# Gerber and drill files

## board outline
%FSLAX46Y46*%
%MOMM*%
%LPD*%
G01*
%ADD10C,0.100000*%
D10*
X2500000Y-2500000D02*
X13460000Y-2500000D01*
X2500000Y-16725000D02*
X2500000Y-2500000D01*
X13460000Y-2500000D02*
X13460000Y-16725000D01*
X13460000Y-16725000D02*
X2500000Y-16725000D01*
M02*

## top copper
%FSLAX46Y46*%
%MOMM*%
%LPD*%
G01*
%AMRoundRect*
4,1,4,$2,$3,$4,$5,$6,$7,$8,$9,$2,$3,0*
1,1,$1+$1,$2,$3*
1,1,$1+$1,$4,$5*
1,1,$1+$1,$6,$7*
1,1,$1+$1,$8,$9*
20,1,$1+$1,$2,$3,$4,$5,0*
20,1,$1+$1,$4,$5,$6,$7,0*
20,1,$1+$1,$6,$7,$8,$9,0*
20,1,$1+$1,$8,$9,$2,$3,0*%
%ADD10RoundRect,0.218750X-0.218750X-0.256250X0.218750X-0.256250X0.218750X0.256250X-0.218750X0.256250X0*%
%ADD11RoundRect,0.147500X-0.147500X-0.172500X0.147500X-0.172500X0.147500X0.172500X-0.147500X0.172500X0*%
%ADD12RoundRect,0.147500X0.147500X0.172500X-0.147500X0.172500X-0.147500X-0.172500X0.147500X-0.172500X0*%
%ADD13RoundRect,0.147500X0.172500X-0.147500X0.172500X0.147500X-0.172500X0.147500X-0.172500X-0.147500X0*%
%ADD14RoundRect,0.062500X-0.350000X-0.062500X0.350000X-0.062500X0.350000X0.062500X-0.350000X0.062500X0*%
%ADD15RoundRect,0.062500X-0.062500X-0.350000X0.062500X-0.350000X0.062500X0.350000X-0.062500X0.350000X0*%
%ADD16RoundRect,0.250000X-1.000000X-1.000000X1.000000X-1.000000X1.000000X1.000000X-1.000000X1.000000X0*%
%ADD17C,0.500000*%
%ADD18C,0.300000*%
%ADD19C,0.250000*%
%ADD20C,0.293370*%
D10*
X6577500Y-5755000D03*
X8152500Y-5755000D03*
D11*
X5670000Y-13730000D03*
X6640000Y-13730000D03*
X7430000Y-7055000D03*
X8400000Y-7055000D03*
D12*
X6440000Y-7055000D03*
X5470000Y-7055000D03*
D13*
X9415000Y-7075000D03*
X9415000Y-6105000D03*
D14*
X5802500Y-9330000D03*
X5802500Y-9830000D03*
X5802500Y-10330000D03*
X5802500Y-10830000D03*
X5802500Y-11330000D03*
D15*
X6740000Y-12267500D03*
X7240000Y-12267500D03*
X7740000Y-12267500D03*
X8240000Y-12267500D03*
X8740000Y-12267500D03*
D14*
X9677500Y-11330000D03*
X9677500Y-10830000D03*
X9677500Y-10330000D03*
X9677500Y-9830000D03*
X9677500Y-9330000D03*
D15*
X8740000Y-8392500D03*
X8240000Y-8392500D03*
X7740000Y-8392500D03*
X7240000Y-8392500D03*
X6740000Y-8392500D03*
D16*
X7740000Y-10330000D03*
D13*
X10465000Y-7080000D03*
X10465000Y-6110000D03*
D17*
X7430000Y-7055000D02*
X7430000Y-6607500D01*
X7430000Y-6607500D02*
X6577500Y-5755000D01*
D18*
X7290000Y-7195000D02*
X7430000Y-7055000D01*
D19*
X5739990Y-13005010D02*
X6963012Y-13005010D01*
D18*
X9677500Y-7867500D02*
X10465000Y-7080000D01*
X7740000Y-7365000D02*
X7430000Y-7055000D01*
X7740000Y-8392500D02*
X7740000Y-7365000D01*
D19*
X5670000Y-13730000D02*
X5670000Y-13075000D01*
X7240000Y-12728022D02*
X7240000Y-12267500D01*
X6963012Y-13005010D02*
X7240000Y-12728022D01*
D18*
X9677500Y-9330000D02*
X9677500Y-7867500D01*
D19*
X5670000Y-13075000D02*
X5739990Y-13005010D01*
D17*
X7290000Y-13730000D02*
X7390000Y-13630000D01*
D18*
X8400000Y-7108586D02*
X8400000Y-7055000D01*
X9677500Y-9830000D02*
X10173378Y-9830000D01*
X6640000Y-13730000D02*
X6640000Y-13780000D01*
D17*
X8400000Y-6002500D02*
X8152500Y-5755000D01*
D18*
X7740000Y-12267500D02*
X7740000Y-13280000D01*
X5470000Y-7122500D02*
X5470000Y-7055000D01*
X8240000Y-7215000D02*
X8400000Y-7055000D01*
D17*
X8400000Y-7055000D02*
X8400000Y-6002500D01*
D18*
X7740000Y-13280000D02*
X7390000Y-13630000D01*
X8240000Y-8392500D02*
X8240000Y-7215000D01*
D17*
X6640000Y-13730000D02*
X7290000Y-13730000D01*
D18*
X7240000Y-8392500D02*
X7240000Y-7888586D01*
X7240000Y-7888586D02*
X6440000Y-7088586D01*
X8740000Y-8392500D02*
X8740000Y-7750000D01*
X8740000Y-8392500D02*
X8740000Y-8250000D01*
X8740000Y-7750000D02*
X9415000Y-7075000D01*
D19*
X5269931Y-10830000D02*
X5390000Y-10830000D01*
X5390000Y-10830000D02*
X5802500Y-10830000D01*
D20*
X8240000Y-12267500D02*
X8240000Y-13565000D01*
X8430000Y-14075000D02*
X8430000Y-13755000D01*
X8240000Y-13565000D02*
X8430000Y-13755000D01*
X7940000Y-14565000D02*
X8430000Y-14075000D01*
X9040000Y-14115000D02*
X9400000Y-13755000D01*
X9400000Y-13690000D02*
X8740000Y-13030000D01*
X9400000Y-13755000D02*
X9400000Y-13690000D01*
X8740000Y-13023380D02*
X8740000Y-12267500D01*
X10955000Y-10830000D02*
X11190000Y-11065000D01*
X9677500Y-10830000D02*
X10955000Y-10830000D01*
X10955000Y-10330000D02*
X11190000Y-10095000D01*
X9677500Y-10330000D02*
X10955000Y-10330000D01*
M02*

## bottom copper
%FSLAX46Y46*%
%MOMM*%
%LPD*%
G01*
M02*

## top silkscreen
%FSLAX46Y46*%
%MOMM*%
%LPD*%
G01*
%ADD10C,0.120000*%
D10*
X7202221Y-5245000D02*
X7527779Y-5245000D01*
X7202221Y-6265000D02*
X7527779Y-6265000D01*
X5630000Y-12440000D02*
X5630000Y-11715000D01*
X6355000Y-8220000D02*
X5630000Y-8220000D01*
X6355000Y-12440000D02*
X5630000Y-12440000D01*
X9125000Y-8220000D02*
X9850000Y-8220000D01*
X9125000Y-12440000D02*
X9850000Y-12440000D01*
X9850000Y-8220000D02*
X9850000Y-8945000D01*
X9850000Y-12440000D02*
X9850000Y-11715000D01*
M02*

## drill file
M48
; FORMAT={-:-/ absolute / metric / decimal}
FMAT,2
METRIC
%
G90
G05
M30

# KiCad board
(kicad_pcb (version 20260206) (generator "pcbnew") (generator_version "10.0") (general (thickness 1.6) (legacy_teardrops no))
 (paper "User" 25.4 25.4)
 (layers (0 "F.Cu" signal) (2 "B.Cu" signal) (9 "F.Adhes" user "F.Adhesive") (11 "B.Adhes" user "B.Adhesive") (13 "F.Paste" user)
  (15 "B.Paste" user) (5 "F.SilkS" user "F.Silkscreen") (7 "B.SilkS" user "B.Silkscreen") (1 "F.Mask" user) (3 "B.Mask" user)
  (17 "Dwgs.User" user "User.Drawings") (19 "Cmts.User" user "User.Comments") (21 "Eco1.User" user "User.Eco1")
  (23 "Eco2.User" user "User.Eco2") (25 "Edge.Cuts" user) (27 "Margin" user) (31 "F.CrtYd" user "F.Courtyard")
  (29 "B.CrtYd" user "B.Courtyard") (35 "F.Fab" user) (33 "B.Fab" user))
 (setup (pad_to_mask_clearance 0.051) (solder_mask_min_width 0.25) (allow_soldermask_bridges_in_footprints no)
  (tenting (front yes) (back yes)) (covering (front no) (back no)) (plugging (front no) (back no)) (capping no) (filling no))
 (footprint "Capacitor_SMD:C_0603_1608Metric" (layer "F.Cu") (at 7.365 5.755)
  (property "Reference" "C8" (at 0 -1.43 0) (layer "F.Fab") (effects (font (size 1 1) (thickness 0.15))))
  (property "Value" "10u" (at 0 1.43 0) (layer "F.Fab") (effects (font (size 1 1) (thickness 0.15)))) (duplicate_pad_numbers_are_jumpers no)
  (fp_line (start -0.162779 -0.51) (end 0.162779 -0.51) (stroke (width 0.12) (type solid)) (layer "F.SilkS"))
  (fp_line (start -0.162779 0.51) (end 0.162779 0.51) (stroke (width 0.12) (type solid)) (layer "F.SilkS"))
  (pad "1" smd roundrect (at -0.7875 0) (size 0.875 0.95) (layers "F.Cu" "F.Mask" "F.Paste") (roundrect_rratio 0.25) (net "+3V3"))
  (pad "2" smd roundrect (at 0.7875 0) (size 0.875 0.95) (layers "F.Cu" "F.Mask" "F.Paste") (roundrect_rratio 0.25) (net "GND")))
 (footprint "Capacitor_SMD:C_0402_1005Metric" (layer "F.Cu") (at 6.155 13.73)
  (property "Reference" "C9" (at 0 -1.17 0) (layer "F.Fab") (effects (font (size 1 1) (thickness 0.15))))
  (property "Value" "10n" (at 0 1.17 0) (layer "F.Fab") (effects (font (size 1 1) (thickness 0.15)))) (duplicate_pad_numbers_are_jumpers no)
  (pad "1" smd roundrect (at -0.485 0) (size 0.59 0.64) (layers "F.Cu" "F.Mask" "F.Paste") (roundrect_rratio 0.25) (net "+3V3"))
  (pad "2" smd roundrect (at 0.485 0) (size 0.59 0.64) (layers "F.Cu" "F.Mask" "F.Paste") (roundrect_rratio 0.25) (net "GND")))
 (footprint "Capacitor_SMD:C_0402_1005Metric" (layer "F.Cu") (at 7.915 7.055)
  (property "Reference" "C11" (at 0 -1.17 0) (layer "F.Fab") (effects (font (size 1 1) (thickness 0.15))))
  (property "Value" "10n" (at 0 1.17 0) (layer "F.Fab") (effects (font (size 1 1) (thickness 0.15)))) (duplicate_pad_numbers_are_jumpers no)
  (pad "1" smd roundrect (at -0.485 0) (size 0.59 0.64) (layers "F.Cu" "F.Mask" "F.Paste") (roundrect_rratio 0.25) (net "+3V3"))
  (pad "2" smd roundrect (at 0.485 0) (size 0.59 0.64) (layers "F.Cu" "F.Mask" "F.Paste") (roundrect_rratio 0.25) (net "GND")))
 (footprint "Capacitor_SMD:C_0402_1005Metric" (layer "F.Cu") (at 5.955 7.055 180)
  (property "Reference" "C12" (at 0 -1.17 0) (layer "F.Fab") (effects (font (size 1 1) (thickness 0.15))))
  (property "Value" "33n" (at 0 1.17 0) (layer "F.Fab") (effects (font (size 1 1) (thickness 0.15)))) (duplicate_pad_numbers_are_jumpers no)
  (pad "1" smd roundrect (at -0.485 0 180) (size 0.59 0.64) (layers "F.Cu" "F.Mask" "F.Paste") (roundrect_rratio 0.25)
   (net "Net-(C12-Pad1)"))
  (pad "2" smd roundrect (at 0.485 0 180) (size 0.59 0.64) (layers "F.Cu" "F.Mask" "F.Paste") (roundrect_rratio 0.25) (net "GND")))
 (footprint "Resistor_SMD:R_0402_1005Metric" (layer "F.Cu") (at 9.415 6.59 90)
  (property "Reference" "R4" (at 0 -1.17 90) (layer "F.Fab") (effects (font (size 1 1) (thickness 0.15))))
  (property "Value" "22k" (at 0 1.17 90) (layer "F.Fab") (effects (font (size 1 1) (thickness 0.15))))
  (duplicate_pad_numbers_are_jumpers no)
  (pad "1" smd roundrect (at -0.485 0 90) (size 0.59 0.64) (layers "F.Cu" "F.Mask" "F.Paste") (roundrect_rratio 0.25) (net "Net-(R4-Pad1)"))
  (pad "2" smd roundrect (at 0.485 0 90) (size 0.59 0.64) (layers "F.Cu" "F.Mask" "F.Paste") (roundrect_rratio 0.25) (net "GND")))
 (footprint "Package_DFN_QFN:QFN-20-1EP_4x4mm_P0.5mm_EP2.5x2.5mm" (layer "F.Cu") (at 7.74 10.33)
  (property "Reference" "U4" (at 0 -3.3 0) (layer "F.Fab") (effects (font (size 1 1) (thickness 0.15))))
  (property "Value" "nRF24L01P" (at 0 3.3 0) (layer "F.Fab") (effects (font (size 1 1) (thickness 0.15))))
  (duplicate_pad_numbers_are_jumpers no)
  (fp_line (start -2.11 2.11) (end -2.11 1.385) (stroke (width 0.12) (type solid)) (layer "F.SilkS"))
  (fp_line (start -1.385 -2.11) (end -2.11 -2.11) (stroke (width 0.12) (type solid)) (layer "F.SilkS"))
  (fp_line (start -1.385 2.11) (end -2.11 2.11) (stroke (width 0.12) (type solid)) (layer "F.SilkS"))
  (fp_line (start 1.385 -2.11) (end 2.11 -2.11) (stroke (width 0.12) (type solid)) (layer "F.SilkS"))
  (fp_line (start 1.385 2.11) (end 2.11 2.11) (stroke (width 0.12) (type solid)) (layer "F.SilkS"))
  (fp_line (start 2.11 -2.11) (end 2.11 -1.385) (stroke (width 0.12) (type solid)) (layer "F.SilkS"))
  (fp_line (start 2.11 2.11) (end 2.11 1.385) (stroke (width 0.12) (type solid)) (layer "F.SilkS"))
  (pad "" smd roundrect (at -0.625 -0.625) (size 1.01 1.01) (layers "F.Paste") (roundrect_rratio 0.247525))
  (pad "" smd roundrect (at -0.625 0.625) (size 1.01 1.01) (layers "F.Paste") (roundrect_rratio 0.247525))
  (pad "" smd roundrect (at 0.625 -0.625) (size 1.01 1.01) (layers "F.Paste") (roundrect_rratio 0.247525))
  (pad "" smd roundrect (at 0.625 0.625) (size 1.01 1.01) (layers "F.Paste") (roundrect_rratio 0.247525))
  (pad "1" smd roundrect (at -1.9375 -1) (size 0.825 0.25) (layers "F.Cu" "F.Mask" "F.Paste") (roundrect_rratio 0.25) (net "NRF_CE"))
  (pad "2" smd roundrect (at -1.9375 -0.5) (size 0.825 0.25) (layers "F.Cu" "F.Mask" "F.Paste") (roundrect_rratio 0.25) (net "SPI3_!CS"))
  (pad "3" smd roundrect (at -1.9375 0) (size 0.825 0.25) (layers "F.Cu" "F.Mask" "F.Paste") (roundrect_rratio 0.25) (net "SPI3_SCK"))
  (pad "4" smd roundrect (at -1.9375 0.5) (size 0.825 0.25) (layers "F.Cu" "F.Mask" "F.Paste") (roundrect_rratio 0.25) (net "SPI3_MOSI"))
  (pad "5" smd roundrect (at -1.9375 1) (size 0.825 0.25) (layers "F.Cu" "F.Mask" "F.Paste") (roundrect_rratio 0.25) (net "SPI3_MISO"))
  (pad "6" smd roundrect (at -1 1.9375) (size 0.25 0.825) (layers "F.Cu" "F.Mask" "F.Paste") (roundrect_rratio 0.25) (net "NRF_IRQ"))
  (pad "7" smd roundrect (at -0.5 1.9375) (size 0.25 0.825) (layers "F.Cu" "F.Mask" "F.Paste") (roundrect_rratio 0.25) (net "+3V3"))
  (pad "8" smd roundrect (at 0 1.9375) (size 0.25 0.825) (layers "F.Cu" "F.Mask" "F.Paste") (roundrect_rratio 0.25) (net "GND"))
  (pad "9" smd roundrect (at 0.5 1.9375) (size 0.25 0.825) (layers "F.Cu" "F.Mask" "F.Paste") (roundrect_rratio 0.25) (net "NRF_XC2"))
  (pad "10" smd roundrect (at 1 1.9375) (size 0.25 0.825) (layers "F.Cu" "F.Mask" "F.Paste") (roundrect_rratio 0.25) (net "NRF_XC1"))
  (pad "11" smd roundrect (at 1.9375 1) (size 0.825 0.25) (layers "F.Cu" "F.Mask" "F.Paste") (roundrect_rratio 0.25) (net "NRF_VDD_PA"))
  (pad "12" smd roundrect (at 1.9375 0.5) (size 0.825 0.25) (layers "F.Cu" "F.Mask" "F.Paste") (roundrect_rratio 0.25) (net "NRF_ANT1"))
  (pad "13" smd roundrect (at 1.9375 0) (size 0.825 0.25) (layers "F.Cu" "F.Mask" "F.Paste") (roundrect_rratio 0.25) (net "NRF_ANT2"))
  (pad "14" smd roundrect (at 1.9375 -0.5) (size 0.825 0.25) (layers "F.Cu" "F.Mask" "F.Paste") (roundrect_rratio 0.25) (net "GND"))
  (pad "15" smd roundrect (at 1.9375 -1) (size 0.825 0.25) (layers "F.Cu" "F.Mask" "F.Paste") (roundrect_rratio 0.25) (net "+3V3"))
  (pad "16" smd roundrect (at 1 -1.9375) (size 0.25 0.825) (layers "F.Cu" "F.Mask" "F.Paste") (roundrect_rratio 0.25) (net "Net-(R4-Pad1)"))
  (pad "17" smd roundrect (at 0.5 -1.9375) (size 0.25 0.825) (layers "F.Cu" "F.Mask" "F.Paste") (roundrect_rratio 0.25) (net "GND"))
  (pad "18" smd roundrect (at 0 -1.9375) (size 0.25 0.825) (layers "F.Cu" "F.Mask" "F.Paste") (roundrect_rratio 0.25) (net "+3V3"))
  (pad "19" smd roundrect (at -0.5 -1.9375) (size 0.25 0.825) (layers "F.Cu" "F.Mask" "F.Paste") (roundrect_rratio 0.25)
   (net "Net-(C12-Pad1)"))
  (pad "20" smd roundrect (at -1 -1.9375) (size 0.25 0.825) (layers "F.Cu" "F.Mask" "F.Paste") (roundrect_rratio 0.25) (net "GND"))
  (pad "21" smd roundrect (at 0 0) (size 2.5 2.5) (layers "F.Cu" "F.Mask") (roundrect_rratio 0.1) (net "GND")))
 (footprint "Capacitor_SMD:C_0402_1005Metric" (layer "F.Cu") (at 10.465 6.595 90)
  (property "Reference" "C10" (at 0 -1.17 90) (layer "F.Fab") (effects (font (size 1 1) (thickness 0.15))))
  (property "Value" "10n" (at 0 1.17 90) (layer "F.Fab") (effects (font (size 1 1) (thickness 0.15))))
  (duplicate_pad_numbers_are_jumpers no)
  (pad "1" smd roundrect (at -0.485 0 90) (size 0.59 0.64) (layers "F.Cu" "F.Mask" "F.Paste") (roundrect_rratio 0.25) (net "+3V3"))
  (pad "2" smd roundrect (at 0.485 0 90) (size 0.59 0.64) (layers "F.Cu" "F.Mask" "F.Paste") (roundrect_rratio 0.25) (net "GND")))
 (gr_line (start 2.5 2.5) (end 13.46 2.5) (stroke (width 0.1) (type default)) (layer "Edge.Cuts"))
 (gr_line (start 2.5 16.725) (end 2.5 2.5) (stroke (width 0.1) (type default)) (layer "Edge.Cuts"))
 (gr_line (start 13.46 2.5) (end 13.46 16.725) (stroke (width 0.1) (type default)) (layer "Edge.Cuts"))
 (gr_line (start 13.46 16.725) (end 2.5 16.725) (stroke (width 0.1) (type default)) (layer "Edge.Cuts"))
 (segment (start 7.43 7.055) (end 7.43 6.6075) (width 0.5) (layer "F.Cu") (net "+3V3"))
 (segment (start 7.43 6.6075) (end 6.5775 5.755) (width 0.5) (layer "F.Cu") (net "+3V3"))
 (segment (start 7.29 7.195) (end 7.43 7.055) (width 0.3) (layer "F.Cu") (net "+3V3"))
 (segment (start 5.73999 13.00501) (end 6.963012 13.00501) (width 0.25) (layer "F.Cu") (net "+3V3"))
 (segment (start 9.6775 7.8675) (end 10.465 7.08) (width 0.3) (layer "F.Cu") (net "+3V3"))
 (segment (start 7.74 7.365) (end 7.43 7.055) (width 0.3) (layer "F.Cu") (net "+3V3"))
 (segment (start 7.74 8.3925) (end 7.74 7.365) (width 0.3) (layer "F.Cu") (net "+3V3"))
 (segment (start 5.67 13.73) (end 5.67 13.075) (width 0.25) (layer "F.Cu") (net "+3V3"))
 (segment (start 7.24 12.728022) (end 7.24 12.2675) (width 0.25) (layer "F.Cu") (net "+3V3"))
 (segment (start 6.963012 13.00501) (end 7.24 12.728022) (width 0.25) (layer "F.Cu") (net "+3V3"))
 (segment (start 9.6775 9.33) (end 9.6775 7.8675) (width 0.3) (layer "F.Cu") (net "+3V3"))
 (segment (start 5.67 13.075) (end 5.73999 13.00501) (width 0.25) (layer "F.Cu") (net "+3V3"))
 (segment (start 7.29 13.73) (end 7.39 13.63) (width 0.5) (layer "F.Cu") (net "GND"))
 (segment (start 8.4 7.108586) (end 8.4 7.055) (width 0.3) (layer "F.Cu") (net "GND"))
 (segment (start 9.6775 9.83) (end 10.173378 9.83) (width 0.3) (layer "F.Cu") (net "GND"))
 (segment (start 6.64 13.73) (end 6.64 13.78) (width 0.3) (layer "F.Cu") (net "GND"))
 (segment (start 8.4 6.0025) (end 8.1525 5.755) (width 0.5) (layer "F.Cu") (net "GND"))
 (segment (start 7.74 12.2675) (end 7.74 13.28) (width 0.3) (layer "F.Cu") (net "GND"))
 (segment (start 5.47 7.1225) (end 5.47 7.055) (width 0.3) (layer "F.Cu") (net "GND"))
 (segment (start 8.24 7.215) (end 8.4 7.055) (width 0.3) (layer "F.Cu") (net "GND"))
 (segment (start 8.4 7.055) (end 8.4 6.0025) (width 0.5) (layer "F.Cu") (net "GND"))
 (segment (start 7.74 13.28) (end 7.39 13.63) (width 0.3) (layer "F.Cu") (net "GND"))
 (segment (start 8.24 8.3925) (end 8.24 7.215) (width 0.3) (layer "F.Cu") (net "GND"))
 (segment (start 6.64 13.73) (end 7.29 13.73) (width 0.5) (layer "F.Cu") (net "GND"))
 (segment (start 7.24 8.3925) (end 7.24 7.888586) (width 0.3) (layer "F.Cu") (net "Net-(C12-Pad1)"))
 (segment (start 7.24 7.888586) (end 6.44 7.088586) (width 0.3) (layer "F.Cu") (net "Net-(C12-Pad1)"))
 (segment (start 8.74 8.3925) (end 8.74 7.75) (width 0.3) (layer "F.Cu") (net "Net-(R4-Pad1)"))
 (segment (start 8.74 8.3925) (end 8.74 8.25) (width 0.3) (layer "F.Cu") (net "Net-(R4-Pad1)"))
 (segment (start 8.74 7.75) (end 9.415 7.075) (width 0.3) (layer "F.Cu") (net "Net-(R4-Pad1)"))
 (segment (start 5.269931 10.83) (end 5.39 10.83) (width 0.25) (layer "F.Cu") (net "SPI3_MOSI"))
 (segment (start 5.39 10.83) (end 5.8025 10.83) (width 0.25) (layer "F.Cu") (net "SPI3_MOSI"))
 (segment (start 8.24 12.2675) (end 8.24 13.565) (width 0.29337) (layer "F.Cu") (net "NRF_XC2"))
 (segment (start 8.43 14.075) (end 8.43 13.755) (width 0.29337) (layer "F.Cu") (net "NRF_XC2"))
 (segment (start 8.24 13.565) (end 8.43 13.755) (width 0.29337) (layer "F.Cu") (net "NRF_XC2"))
 (segment (start 7.94 14.565) (end 8.43 14.075) (width 0.29337) (layer "F.Cu") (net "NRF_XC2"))
 (segment (start 9.04 14.115) (end 9.4 13.755) (width 0.29337) (layer "F.Cu") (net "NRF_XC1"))
 (segment (start 9.4 13.69) (end 8.74 13.03) (width 0.29337) (layer "F.Cu") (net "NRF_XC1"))
 (segment (start 9.4 13.755) (end 9.4 13.69) (width 0.29337) (layer "F.Cu") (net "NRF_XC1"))
 (segment (start 8.74 13.02338) (end 8.74 12.2675) (width 0.29337) (layer "F.Cu") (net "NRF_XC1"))
 (segment (start 10.955 10.83) (end 11.19 11.065) (width 0.29337) (layer "F.Cu") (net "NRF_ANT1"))
 (segment (start 9.6775 10.83) (end 10.955 10.83) (width 0.29337) (layer "F.Cu") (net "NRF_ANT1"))
 (segment (start 10.955 10.33) (end 11.19 10.095) (width 0.29337) (layer "F.Cu") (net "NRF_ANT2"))
 (segment (start 9.6775 10.33) (end 10.955 10.33) (width 0.29337) (layer "F.Cu") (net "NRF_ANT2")))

